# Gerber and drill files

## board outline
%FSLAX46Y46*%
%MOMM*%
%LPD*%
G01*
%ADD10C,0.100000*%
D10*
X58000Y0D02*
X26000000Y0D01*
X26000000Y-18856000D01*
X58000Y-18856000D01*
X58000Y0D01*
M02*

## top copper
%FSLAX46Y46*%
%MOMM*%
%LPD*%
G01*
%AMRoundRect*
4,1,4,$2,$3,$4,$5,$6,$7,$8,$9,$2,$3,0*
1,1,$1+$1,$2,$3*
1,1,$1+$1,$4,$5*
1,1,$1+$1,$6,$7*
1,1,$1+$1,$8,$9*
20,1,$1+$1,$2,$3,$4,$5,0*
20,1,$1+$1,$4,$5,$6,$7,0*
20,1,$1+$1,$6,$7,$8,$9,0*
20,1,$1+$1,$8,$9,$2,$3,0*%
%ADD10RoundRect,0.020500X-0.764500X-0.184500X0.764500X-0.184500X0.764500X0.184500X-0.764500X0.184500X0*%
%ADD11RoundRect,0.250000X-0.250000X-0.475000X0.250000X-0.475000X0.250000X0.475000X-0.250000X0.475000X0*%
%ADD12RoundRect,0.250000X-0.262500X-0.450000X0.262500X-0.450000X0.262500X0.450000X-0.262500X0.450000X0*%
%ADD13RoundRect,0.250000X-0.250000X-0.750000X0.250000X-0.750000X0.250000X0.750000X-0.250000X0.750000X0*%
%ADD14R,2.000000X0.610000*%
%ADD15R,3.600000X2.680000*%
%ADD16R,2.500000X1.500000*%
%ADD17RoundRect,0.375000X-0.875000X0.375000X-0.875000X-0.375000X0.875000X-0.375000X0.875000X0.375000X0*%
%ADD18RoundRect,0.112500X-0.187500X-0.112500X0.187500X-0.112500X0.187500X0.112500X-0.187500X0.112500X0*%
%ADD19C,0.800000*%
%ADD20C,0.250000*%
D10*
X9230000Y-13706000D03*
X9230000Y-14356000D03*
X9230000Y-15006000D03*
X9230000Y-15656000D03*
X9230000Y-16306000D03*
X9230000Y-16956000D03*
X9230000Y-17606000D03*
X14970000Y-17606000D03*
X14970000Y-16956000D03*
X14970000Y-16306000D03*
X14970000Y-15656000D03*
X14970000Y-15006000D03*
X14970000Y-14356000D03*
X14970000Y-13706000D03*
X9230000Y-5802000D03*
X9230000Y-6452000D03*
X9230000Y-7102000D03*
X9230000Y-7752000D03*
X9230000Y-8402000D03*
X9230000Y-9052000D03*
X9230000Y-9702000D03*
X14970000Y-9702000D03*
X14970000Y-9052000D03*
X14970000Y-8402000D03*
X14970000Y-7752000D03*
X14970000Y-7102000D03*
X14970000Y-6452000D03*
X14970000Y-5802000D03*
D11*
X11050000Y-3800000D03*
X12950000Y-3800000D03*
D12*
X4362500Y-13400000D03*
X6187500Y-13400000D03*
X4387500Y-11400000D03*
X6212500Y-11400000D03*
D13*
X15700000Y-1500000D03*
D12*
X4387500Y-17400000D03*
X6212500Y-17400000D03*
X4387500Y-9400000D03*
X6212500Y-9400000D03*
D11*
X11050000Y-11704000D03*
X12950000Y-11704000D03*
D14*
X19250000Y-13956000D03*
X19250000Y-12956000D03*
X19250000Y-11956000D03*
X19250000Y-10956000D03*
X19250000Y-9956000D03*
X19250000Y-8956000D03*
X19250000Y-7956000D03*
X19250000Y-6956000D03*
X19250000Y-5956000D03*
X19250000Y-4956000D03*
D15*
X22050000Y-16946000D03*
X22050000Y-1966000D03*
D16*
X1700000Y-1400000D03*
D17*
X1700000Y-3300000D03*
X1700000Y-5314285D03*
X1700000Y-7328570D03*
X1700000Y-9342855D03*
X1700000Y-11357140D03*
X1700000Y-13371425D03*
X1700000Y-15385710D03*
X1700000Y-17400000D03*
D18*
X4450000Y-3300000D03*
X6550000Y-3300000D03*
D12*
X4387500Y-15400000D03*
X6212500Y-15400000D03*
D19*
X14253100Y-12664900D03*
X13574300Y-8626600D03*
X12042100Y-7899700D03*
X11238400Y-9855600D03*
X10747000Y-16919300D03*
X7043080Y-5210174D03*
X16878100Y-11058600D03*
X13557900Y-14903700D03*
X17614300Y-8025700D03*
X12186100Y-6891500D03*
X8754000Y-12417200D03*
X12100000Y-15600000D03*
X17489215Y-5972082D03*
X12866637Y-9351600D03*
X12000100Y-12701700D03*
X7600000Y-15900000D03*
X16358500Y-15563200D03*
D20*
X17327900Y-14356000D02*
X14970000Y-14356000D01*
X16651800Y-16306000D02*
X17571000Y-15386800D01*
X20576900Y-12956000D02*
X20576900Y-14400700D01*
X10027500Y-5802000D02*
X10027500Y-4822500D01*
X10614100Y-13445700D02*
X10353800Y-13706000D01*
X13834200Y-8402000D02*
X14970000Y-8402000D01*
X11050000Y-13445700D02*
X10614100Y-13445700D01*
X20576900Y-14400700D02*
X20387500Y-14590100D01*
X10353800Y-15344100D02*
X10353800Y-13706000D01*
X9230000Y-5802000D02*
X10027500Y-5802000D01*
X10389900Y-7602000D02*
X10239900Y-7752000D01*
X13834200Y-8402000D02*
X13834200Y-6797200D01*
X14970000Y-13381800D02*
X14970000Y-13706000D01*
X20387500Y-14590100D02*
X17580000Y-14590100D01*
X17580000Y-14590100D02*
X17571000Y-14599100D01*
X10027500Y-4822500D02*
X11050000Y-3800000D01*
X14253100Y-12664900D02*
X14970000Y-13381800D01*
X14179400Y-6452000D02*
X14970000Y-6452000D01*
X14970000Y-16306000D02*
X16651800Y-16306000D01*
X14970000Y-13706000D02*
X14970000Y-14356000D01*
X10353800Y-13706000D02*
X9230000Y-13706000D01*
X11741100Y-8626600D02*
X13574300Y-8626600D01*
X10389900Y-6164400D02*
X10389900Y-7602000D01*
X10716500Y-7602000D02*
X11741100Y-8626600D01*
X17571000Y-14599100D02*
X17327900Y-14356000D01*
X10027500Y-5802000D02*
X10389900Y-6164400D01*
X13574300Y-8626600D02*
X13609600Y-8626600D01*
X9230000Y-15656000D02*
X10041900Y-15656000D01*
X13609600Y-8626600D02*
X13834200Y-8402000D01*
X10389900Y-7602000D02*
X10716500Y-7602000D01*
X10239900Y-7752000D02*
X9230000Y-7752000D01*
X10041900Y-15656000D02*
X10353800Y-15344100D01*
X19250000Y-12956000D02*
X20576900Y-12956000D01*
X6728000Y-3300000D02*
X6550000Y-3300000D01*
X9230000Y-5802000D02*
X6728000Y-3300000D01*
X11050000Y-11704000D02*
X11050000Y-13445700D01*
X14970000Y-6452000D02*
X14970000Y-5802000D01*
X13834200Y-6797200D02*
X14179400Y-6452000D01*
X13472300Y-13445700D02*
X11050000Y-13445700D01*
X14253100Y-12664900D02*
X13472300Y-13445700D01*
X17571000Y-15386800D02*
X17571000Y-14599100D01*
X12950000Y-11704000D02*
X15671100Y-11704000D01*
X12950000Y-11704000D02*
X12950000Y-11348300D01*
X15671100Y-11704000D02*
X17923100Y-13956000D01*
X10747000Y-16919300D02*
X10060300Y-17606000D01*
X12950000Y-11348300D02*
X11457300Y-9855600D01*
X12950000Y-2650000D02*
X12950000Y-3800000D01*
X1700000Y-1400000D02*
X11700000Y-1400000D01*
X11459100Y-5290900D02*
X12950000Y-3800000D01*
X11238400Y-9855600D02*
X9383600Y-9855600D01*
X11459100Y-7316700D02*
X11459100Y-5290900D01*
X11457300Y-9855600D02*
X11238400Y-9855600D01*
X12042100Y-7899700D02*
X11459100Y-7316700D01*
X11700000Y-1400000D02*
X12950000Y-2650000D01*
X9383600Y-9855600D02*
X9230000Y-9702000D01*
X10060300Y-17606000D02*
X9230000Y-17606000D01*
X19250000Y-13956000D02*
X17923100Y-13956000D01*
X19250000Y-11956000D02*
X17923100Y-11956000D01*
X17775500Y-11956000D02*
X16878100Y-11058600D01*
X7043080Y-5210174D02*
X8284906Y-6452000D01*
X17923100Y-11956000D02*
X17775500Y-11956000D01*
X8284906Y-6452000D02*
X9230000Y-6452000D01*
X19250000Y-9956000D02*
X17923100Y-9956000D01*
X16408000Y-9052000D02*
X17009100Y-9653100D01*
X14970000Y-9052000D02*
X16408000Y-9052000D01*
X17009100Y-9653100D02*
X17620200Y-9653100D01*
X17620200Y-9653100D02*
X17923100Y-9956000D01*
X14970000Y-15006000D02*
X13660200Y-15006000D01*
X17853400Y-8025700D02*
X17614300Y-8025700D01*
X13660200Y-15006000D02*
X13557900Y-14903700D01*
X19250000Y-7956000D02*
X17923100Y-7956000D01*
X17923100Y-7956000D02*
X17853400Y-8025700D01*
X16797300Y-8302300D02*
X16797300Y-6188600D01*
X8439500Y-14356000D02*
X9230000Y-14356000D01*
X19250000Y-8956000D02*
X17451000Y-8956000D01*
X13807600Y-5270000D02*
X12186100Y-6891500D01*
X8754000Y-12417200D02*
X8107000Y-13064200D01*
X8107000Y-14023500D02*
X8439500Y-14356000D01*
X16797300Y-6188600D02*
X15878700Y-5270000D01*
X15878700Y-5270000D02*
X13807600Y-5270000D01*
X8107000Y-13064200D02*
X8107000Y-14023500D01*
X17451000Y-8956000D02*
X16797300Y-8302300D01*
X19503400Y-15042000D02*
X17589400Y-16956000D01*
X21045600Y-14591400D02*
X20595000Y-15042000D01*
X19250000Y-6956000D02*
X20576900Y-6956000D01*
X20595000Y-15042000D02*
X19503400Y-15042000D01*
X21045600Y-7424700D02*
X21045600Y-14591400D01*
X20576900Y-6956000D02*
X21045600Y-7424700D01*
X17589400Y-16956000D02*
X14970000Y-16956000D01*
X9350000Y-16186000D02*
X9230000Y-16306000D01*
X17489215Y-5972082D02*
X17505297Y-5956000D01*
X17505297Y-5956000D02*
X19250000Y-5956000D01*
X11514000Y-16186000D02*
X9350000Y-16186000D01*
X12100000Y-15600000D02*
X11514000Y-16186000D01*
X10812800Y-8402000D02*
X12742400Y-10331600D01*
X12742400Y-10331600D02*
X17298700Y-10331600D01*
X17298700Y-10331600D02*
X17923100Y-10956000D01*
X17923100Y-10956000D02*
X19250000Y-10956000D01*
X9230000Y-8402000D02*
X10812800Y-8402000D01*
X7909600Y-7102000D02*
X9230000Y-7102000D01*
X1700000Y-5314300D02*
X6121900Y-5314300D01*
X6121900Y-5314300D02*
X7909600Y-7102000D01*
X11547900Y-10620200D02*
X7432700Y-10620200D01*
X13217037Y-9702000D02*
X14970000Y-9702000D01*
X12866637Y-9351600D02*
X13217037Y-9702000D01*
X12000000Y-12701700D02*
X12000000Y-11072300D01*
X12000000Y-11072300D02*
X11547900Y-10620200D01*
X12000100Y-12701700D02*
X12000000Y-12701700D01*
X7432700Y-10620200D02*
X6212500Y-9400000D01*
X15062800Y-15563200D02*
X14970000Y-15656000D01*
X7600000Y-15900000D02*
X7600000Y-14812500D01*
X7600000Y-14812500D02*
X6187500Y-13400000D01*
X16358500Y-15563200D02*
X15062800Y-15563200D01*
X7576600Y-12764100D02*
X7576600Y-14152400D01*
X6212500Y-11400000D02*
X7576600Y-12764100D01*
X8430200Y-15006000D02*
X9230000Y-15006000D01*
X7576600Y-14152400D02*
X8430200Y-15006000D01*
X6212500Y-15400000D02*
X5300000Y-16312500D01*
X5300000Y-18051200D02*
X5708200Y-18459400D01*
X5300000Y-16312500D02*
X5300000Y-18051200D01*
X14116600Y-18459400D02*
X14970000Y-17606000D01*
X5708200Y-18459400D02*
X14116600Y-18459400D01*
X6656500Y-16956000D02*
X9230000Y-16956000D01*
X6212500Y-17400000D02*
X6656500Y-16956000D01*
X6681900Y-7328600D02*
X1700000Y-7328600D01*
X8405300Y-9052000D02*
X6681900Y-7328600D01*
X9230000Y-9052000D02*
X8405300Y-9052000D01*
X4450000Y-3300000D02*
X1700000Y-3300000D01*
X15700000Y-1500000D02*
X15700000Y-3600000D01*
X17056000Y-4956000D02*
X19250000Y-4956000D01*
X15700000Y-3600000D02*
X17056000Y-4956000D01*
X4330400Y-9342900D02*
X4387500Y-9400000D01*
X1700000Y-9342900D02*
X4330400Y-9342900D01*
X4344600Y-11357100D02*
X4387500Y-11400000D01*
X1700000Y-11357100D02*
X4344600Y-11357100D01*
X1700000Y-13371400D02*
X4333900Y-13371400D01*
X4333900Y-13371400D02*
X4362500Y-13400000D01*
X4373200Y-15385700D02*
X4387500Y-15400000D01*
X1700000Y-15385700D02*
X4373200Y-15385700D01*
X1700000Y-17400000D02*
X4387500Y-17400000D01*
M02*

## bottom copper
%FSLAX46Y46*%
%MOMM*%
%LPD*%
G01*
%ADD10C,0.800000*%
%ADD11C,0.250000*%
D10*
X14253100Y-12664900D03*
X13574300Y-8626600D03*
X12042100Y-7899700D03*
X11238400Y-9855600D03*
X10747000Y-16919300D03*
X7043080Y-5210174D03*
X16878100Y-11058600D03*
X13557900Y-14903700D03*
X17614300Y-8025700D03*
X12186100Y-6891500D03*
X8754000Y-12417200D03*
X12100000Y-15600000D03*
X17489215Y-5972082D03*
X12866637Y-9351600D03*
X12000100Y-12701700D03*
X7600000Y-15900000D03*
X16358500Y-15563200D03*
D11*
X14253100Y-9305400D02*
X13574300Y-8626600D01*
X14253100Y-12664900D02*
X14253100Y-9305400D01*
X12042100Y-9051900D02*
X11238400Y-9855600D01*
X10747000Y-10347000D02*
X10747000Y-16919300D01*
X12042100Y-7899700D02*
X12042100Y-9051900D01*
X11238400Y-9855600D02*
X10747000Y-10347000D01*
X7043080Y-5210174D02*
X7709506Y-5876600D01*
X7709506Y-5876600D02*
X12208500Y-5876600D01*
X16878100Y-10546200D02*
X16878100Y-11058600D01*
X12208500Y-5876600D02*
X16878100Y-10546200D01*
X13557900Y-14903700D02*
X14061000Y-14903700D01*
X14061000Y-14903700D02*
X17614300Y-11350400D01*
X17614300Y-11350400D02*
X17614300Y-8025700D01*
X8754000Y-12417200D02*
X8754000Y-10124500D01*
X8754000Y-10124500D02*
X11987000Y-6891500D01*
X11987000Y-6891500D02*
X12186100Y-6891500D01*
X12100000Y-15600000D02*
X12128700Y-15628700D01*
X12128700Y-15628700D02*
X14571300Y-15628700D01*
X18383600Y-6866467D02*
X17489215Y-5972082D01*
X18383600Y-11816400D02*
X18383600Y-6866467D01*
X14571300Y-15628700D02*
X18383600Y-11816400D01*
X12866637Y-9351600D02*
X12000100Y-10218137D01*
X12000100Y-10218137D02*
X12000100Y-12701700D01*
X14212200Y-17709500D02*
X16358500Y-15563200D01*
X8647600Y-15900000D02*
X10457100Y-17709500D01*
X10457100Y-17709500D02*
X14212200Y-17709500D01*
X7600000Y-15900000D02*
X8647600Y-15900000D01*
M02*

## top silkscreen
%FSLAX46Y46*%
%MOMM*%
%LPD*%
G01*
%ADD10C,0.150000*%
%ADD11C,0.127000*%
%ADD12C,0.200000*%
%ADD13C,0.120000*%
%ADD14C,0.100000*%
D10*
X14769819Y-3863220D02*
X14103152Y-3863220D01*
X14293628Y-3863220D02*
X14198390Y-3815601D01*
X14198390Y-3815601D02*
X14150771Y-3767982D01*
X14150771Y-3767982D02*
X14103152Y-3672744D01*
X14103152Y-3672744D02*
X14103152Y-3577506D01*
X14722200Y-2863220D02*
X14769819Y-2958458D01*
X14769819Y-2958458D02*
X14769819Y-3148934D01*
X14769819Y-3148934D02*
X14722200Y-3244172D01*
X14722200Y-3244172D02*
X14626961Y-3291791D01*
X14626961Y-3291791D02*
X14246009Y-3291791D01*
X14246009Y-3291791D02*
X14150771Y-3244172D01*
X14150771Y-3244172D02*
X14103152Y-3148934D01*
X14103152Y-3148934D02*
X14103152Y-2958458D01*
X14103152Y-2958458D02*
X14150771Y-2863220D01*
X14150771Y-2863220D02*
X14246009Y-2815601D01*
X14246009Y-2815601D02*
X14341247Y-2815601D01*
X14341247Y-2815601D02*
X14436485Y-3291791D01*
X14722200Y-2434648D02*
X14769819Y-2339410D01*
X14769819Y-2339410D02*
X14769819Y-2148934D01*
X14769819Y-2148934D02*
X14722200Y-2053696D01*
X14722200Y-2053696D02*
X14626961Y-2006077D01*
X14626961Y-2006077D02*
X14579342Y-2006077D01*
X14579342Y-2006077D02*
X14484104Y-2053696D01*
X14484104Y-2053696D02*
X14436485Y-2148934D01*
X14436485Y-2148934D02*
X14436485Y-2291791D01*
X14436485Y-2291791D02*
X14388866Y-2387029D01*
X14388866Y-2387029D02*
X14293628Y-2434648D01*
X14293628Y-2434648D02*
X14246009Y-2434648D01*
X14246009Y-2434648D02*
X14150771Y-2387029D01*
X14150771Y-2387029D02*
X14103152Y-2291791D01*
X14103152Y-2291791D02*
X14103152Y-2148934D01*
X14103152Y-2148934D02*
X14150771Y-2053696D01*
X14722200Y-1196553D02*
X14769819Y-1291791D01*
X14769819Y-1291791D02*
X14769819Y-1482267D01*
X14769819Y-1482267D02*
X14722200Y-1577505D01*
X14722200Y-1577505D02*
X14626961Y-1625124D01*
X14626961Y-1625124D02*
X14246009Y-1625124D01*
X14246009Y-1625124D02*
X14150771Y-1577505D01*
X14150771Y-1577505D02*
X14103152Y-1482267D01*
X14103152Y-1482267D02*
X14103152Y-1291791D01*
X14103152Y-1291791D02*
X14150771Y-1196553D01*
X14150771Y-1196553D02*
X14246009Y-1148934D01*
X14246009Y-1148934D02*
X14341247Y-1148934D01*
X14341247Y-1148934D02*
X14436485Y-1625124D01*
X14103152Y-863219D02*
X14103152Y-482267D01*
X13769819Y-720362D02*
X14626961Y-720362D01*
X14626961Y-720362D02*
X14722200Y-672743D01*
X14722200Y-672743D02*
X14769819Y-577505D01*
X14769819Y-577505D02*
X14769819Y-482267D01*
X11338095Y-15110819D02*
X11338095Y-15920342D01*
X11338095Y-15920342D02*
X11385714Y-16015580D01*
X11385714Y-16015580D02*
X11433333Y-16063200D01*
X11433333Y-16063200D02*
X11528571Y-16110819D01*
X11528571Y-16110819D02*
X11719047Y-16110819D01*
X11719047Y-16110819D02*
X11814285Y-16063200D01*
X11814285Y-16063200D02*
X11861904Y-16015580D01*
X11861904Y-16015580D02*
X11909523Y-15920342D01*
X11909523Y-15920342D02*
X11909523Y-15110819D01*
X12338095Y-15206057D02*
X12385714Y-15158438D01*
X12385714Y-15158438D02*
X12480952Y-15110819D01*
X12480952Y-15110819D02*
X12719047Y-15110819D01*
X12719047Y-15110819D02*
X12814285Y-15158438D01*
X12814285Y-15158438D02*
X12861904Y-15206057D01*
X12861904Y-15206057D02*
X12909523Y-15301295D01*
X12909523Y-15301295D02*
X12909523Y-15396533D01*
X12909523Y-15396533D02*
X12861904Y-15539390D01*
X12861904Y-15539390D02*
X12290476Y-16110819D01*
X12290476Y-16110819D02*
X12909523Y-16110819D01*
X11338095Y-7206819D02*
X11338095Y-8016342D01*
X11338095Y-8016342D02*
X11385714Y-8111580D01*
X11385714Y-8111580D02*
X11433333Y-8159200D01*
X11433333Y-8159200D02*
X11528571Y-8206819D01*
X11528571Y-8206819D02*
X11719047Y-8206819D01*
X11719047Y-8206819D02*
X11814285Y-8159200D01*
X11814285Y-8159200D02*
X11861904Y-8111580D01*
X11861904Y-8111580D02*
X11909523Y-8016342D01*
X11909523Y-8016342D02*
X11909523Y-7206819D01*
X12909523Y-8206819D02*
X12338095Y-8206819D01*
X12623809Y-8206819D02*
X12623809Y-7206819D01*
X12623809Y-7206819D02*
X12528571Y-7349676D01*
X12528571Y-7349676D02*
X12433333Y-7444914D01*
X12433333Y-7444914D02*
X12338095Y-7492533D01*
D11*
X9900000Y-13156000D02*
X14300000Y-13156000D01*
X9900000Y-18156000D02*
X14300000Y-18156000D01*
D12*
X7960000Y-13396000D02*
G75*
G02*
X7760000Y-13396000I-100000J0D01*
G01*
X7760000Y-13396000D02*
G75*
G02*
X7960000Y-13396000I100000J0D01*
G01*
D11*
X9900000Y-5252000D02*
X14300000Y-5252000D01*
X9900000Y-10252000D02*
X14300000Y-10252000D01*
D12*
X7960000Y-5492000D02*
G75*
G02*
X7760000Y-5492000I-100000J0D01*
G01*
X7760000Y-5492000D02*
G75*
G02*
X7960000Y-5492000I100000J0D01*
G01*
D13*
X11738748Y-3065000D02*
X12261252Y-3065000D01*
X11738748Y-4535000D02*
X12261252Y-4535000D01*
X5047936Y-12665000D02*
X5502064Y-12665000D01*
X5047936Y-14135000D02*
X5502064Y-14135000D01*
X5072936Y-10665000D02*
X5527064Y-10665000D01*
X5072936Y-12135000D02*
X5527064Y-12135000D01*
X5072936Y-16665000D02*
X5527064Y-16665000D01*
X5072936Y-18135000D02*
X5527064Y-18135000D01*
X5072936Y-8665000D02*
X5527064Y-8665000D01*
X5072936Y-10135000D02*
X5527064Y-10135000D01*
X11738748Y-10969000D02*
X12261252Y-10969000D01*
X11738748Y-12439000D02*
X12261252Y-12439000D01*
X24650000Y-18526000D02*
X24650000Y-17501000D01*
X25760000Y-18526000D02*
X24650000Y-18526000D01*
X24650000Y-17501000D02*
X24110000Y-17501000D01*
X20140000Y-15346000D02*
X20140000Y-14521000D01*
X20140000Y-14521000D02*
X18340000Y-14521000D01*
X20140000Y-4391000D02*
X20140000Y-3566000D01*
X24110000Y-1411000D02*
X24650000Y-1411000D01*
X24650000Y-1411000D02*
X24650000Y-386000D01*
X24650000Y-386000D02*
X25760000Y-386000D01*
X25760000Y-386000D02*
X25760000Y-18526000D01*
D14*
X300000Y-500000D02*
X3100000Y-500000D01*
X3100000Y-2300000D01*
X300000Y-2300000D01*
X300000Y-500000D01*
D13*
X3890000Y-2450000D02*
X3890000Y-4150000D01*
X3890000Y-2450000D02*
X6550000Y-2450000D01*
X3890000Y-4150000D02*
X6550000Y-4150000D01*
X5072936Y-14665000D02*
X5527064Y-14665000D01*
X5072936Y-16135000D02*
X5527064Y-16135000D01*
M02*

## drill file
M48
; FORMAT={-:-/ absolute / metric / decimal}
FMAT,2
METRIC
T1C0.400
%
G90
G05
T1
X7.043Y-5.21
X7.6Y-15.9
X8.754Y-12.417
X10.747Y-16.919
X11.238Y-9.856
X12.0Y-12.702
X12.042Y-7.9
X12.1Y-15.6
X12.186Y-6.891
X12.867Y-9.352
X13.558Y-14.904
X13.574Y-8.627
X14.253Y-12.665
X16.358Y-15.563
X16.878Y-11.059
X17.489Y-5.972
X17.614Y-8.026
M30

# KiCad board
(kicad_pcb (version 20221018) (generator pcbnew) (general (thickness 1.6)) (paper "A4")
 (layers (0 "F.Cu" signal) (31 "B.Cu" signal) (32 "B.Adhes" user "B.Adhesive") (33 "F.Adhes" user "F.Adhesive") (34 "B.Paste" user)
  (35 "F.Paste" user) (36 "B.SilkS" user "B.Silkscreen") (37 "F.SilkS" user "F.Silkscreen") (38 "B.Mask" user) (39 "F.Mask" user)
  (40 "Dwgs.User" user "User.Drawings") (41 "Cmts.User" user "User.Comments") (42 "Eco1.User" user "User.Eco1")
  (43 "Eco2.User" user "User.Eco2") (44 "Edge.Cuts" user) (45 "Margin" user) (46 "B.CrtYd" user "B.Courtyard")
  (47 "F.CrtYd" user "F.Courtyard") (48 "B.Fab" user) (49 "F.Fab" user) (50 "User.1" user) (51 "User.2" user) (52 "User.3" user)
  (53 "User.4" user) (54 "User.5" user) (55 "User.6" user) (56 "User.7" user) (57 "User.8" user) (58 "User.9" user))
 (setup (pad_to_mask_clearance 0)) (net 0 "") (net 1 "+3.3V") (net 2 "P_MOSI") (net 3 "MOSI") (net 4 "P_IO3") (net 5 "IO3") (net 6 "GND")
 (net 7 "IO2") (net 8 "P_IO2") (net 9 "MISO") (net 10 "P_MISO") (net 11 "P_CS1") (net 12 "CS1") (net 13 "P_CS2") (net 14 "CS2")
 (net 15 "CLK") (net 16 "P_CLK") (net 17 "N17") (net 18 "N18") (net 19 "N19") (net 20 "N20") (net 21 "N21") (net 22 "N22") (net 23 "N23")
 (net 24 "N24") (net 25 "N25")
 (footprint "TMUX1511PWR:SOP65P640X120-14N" (layer "F.Cu") (at 12.1 15.656)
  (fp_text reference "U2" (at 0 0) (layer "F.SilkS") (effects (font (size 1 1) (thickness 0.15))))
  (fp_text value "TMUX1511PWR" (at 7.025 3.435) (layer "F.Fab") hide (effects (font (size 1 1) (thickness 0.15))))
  (fp_line (start -2.2 -2.5) (end 2.2 -2.5) (stroke (width 0.127) (type solid)) (layer "F.SilkS"))
  (fp_line (start -2.2 2.5) (end 2.2 2.5) (stroke (width 0.127) (type solid)) (layer "F.SilkS"))
  (fp_circle (center -4.24 -2.26) (end -4.14 -2.26) (stroke (width 0.2) (type solid)) (fill none) (layer "F.SilkS"))
  (pad "1" smd roundrect (at -2.87 -1.95) (size 1.57 0.41) (layers "F.Cu" "F.Paste" "F.Mask") (roundrect_rratio 0.05) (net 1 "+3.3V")
   (solder_mask_margin 0.102))
  (pad "2" smd roundrect (at -2.87 -1.3) (size 1.57 0.41) (layers "F.Cu" "F.Paste" "F.Mask") (roundrect_rratio 0.05) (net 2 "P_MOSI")
   (solder_mask_margin 0.102))
  (pad "3" smd roundrect (at -2.87 -0.65) (size 1.57 0.41) (layers "F.Cu" "F.Paste" "F.Mask") (roundrect_rratio 0.05) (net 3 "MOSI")
   (solder_mask_margin 0.102))
  (pad "4" smd roundrect (at -2.87 0) (size 1.57 0.41) (layers "F.Cu" "F.Paste" "F.Mask") (roundrect_rratio 0.05) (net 1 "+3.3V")
   (solder_mask_margin 0.102))
  (pad "5" smd roundrect (at -2.87 0.65) (size 1.57 0.41) (layers "F.Cu" "F.Paste" "F.Mask") (roundrect_rratio 0.05) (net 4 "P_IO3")
   (solder_mask_margin 0.102))
  (pad "6" smd roundrect (at -2.87 1.3) (size 1.57 0.41) (layers "F.Cu" "F.Paste" "F.Mask") (roundrect_rratio 0.05) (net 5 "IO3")
   (solder_mask_margin 0.102))
  (pad "7" smd roundrect (at -2.87 1.95) (size 1.57 0.41) (layers "F.Cu" "F.Paste" "F.Mask") (roundrect_rratio 0.05) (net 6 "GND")
   (solder_mask_margin 0.102))
  (pad "8" smd roundrect (at 2.87 1.95) (size 1.57 0.41) (layers "F.Cu" "F.Paste" "F.Mask") (roundrect_rratio 0.05) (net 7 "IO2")
   (solder_mask_margin 0.102))
  (pad "9" smd roundrect (at 2.87 1.3) (size 1.57 0.41) (layers "F.Cu" "F.Paste" "F.Mask") (roundrect_rratio 0.05) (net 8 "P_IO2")
   (solder_mask_margin 0.102))
  (pad "10" smd roundrect (at 2.87 0.65) (size 1.57 0.41) (layers "F.Cu" "F.Paste" "F.Mask") (roundrect_rratio 0.05) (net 1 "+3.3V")
   (solder_mask_margin 0.102))
  (pad "11" smd roundrect (at 2.87 0) (size 1.57 0.41) (layers "F.Cu" "F.Paste" "F.Mask") (roundrect_rratio 0.05) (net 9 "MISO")
   (solder_mask_margin 0.102))
  (pad "12" smd roundrect (at 2.87 -0.65) (size 1.57 0.41) (layers "F.Cu" "F.Paste" "F.Mask") (roundrect_rratio 0.05) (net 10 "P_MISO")
   (solder_mask_margin 0.102))
  (pad "13" smd roundrect (at 2.87 -1.3) (size 1.57 0.41) (layers "F.Cu" "F.Paste" "F.Mask") (roundrect_rratio 0.05) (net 1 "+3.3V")
   (solder_mask_margin 0.102))
  (pad "14" smd roundrect (at 2.87 -1.95) (size 1.57 0.41) (layers "F.Cu" "F.Paste" "F.Mask") (roundrect_rratio 0.05) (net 1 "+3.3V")
   (solder_mask_margin 0.102)))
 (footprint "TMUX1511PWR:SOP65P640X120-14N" (layer "F.Cu") (at 12.1 7.752)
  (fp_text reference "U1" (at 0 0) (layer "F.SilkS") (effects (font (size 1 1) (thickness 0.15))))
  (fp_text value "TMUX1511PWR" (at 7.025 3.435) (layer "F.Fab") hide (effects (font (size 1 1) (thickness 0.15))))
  (fp_line (start -2.2 -2.5) (end 2.2 -2.5) (stroke (width 0.127) (type solid)) (layer "F.SilkS"))
  (fp_line (start -2.2 2.5) (end 2.2 2.5) (stroke (width 0.127) (type solid)) (layer "F.SilkS"))
  (fp_circle (center -4.24 -2.26) (end -4.14 -2.26) (stroke (width 0.2) (type solid)) (fill none) (layer "F.SilkS"))
  (pad "1" smd roundrect (at -2.87 -1.95) (size 1.57 0.41) (layers "F.Cu" "F.Paste" "F.Mask") (roundrect_rratio 0.05) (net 1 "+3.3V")
   (solder_mask_margin 0.102))
  (pad "2" smd roundrect (at -2.87 -1.3) (size 1.57 0.41) (layers "F.Cu" "F.Paste" "F.Mask") (roundrect_rratio 0.05) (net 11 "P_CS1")
   (solder_mask_margin 0.102))
  (pad "3" smd roundrect (at -2.87 -0.65) (size 1.57 0.41) (layers "F.Cu" "F.Paste" "F.Mask") (roundrect_rratio 0.05) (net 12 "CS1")
   (solder_mask_margin 0.102))
  (pad "4" smd roundrect (at -2.87 0) (size 1.57 0.41) (layers "F.Cu" "F.Paste" "F.Mask") (roundrect_rratio 0.05) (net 1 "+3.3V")
   (solder_mask_margin 0.102))
  (pad "5" smd roundrect (at -2.87 0.65) (size 1.57 0.41) (layers "F.Cu" "F.Paste" "F.Mask") (roundrect_rratio 0.05) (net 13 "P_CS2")
   (solder_mask_margin 0.102))
  (pad "6" smd roundrect (at -2.87 1.3) (size 1.57 0.41) (layers "F.Cu" "F.Paste" "F.Mask") (roundrect_rratio 0.05) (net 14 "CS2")
   (solder_mask_margin 0.102))
  (pad "7" smd roundrect (at -2.87 1.95) (size 1.57 0.41) (layers "F.Cu" "F.Paste" "F.Mask") (roundrect_rratio 0.05) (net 6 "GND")
   (solder_mask_margin 0.102))
  (pad "8" smd roundrect (at 2.87 1.95) (size 1.57 0.41) (layers "F.Cu" "F.Paste" "F.Mask") (roundrect_rratio 0.05) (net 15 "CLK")
   (solder_mask_margin 0.102))
  (pad "9" smd roundrect (at 2.87 1.3) (size 1.57 0.41) (layers "F.Cu" "F.Paste" "F.Mask") (roundrect_rratio 0.05) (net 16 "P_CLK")
   (solder_mask_margin 0.102))
  (pad "10" smd roundrect (at 2.87 0.65) (size 1.57 0.41) (layers "F.Cu" "F.Paste" "F.Mask") (roundrect_rratio 0.05) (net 1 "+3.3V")
   (solder_mask_margin 0.102))
  (pad "11" smd roundrect (at 2.87 0) (size 1.57 0.41) (layers "F.Cu" "F.Paste" "F.Mask") (roundrect_rratio 0.05) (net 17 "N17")
   (solder_mask_margin 0.102))
  (pad "12" smd roundrect (at 2.87 -0.65) (size 1.57 0.41) (layers "F.Cu" "F.Paste" "F.Mask") (roundrect_rratio 0.05) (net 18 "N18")
   (solder_mask_margin 0.102))
  (pad "13" smd roundrect (at 2.87 -1.3) (size 1.57 0.41) (layers "F.Cu" "F.Paste" "F.Mask") (roundrect_rratio 0.05) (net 1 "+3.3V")
   (solder_mask_margin 0.102))
  (pad "14" smd roundrect (at 2.87 -1.95) (size 1.57 0.41) (layers "F.Cu" "F.Paste" "F.Mask") (roundrect_rratio 0.05) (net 1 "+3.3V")
   (solder_mask_margin 0.102)))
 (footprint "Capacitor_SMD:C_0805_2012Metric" (layer "F.Cu") (at 12 3.8)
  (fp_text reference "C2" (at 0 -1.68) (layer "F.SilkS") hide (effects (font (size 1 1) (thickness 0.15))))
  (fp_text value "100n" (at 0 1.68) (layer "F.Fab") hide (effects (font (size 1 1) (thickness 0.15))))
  (fp_line (start -0.261252 -0.735) (end 0.261252 -0.735) (stroke (width 0.12) (type solid)) (layer "F.SilkS"))
  (fp_line (start -0.261252 0.735) (end 0.261252 0.735) (stroke (width 0.12) (type solid)) (layer "F.SilkS"))
  (pad "1" smd roundrect (at -0.95 0) (size 1 1.45) (layers "F.Cu" "F.Paste" "F.Mask") (roundrect_rratio 0.25) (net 1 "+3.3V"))
  (pad "2" smd roundrect (at 0.95 0) (size 1 1.45) (layers "F.Cu" "F.Paste" "F.Mask") (roundrect_rratio 0.25) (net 6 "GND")))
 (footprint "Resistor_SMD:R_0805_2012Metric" (layer "F.Cu") (at 5.275 13.4)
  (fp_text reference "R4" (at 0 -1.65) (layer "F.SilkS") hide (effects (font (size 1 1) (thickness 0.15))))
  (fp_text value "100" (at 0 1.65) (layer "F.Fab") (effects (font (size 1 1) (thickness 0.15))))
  (fp_line (start -0.227064 -0.735) (end 0.227064 -0.735) (stroke (width 0.12) (type solid)) (layer "F.SilkS"))
  (fp_line (start -0.227064 0.735) (end 0.227064 0.735) (stroke (width 0.12) (type solid)) (layer "F.SilkS"))
  (pad "1" smd roundrect (at -0.9125 0) (size 1.025 1.4) (layers "F.Cu" "F.Paste" "F.Mask") (roundrect_rratio 0.243902439) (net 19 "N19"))
  (pad "2" smd roundrect (at 0.9125 0) (size 1.025 1.4) (layers "F.Cu" "F.Paste" "F.Mask") (roundrect_rratio 0.243902439) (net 9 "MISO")))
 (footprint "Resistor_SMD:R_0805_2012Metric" (layer "F.Cu") (at 5.3 11.4)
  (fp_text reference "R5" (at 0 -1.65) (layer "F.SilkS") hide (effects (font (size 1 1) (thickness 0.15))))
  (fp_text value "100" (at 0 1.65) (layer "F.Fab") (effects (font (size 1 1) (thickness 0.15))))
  (fp_line (start -0.227064 -0.735) (end 0.227064 -0.735) (stroke (width 0.12) (type solid)) (layer "F.SilkS"))
  (fp_line (start -0.227064 0.735) (end 0.227064 0.735) (stroke (width 0.12) (type solid)) (layer "F.SilkS"))
  (pad "1" smd roundrect (at -0.9125 0) (size 1.025 1.4) (layers "F.Cu" "F.Paste" "F.Mask") (roundrect_rratio 0.243902439) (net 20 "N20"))
  (pad "2" smd roundrect (at 0.9125 0) (size 1.025 1.4) (layers "F.Cu" "F.Paste" "F.Mask") (roundrect_rratio 0.243902439) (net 3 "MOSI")))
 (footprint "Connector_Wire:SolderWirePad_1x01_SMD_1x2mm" (layer "F.Cu") (at 15.7 1.5)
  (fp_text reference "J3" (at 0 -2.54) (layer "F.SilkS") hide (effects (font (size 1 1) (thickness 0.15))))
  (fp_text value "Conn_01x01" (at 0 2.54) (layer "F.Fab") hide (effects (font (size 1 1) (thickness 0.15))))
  (pad "1" smd roundrect (at 0 0) (size 1 2) (layers "F.Cu" "F.Paste" "F.Mask") (roundrect_rratio 0.25) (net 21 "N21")))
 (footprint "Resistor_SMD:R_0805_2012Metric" (layer "F.Cu") (at 5.3 17.4)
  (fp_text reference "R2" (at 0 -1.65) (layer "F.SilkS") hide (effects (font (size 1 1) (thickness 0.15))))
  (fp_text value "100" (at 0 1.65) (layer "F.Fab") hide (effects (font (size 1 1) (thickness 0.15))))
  (fp_line (start -0.227064 -0.735) (end 0.227064 -0.735) (stroke (width 0.12) (type solid)) (layer "F.SilkS"))
  (fp_line (start -0.227064 0.735) (end 0.227064 0.735) (stroke (width 0.12) (type solid)) (layer "F.SilkS"))
  (pad "1" smd roundrect (at -0.9125 0) (size 1.025 1.4) (layers "F.Cu" "F.Paste" "F.Mask") (roundrect_rratio 0.243902439) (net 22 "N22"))
  (pad "2" smd roundrect (at 0.9125 0) (size 1.025 1.4) (layers "F.Cu" "F.Paste" "F.Mask") (roundrect_rratio 0.243902439) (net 5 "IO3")))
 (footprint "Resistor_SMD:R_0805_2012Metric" (layer "F.Cu") (at 5.3 9.4)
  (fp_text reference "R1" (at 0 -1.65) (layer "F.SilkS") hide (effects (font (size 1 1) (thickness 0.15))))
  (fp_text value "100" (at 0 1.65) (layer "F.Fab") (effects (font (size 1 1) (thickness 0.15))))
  (fp_line (start -0.227064 -0.735) (end 0.227064 -0.735) (stroke (width 0.12) (type solid)) (layer "F.SilkS"))
  (fp_line (start -0.227064 0.735) (end 0.227064 0.735) (stroke (width 0.12) (type solid)) (layer "F.SilkS"))
  (pad "1" smd roundrect (at -0.9125 0) (size 1.025 1.4) (layers "F.Cu" "F.Paste" "F.Mask") (roundrect_rratio 0.243902439) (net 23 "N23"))
  (pad "2" smd roundrect (at 0.9125 0) (size 1.025 1.4) (layers "F.Cu" "F.Paste" "F.Mask") (roundrect_rratio 0.243902439) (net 15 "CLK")))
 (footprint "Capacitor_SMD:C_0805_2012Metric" (layer "F.Cu") (at 12 11.704)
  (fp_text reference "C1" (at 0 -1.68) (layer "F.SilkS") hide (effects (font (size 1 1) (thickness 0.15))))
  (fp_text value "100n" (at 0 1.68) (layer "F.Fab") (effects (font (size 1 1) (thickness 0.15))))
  (fp_line (start -0.261252 -0.735) (end 0.261252 -0.735) (stroke (width 0.12) (type solid)) (layer "F.SilkS"))
  (fp_line (start -0.261252 0.735) (end 0.261252 0.735) (stroke (width 0.12) (type solid)) (layer "F.SilkS"))
  (pad "1" smd roundrect (at -0.95 0) (size 1 1.45) (layers "F.Cu" "F.Paste" "F.Mask") (roundrect_rratio 0.25) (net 1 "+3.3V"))
  (pad "2" smd roundrect (at 0.95 0) (size 1 1.45) (layers "F.Cu" "F.Paste" "F.Mask") (roundrect_rratio 0.25) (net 6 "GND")))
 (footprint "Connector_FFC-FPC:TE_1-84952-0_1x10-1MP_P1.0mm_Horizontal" (layer "F.Cu") (at 21.05 9.456 90)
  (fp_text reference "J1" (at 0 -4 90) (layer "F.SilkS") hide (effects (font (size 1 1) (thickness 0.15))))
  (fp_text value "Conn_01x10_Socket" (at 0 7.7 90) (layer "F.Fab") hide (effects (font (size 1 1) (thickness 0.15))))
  (fp_line (start -9.07 3.6) (end -8.045 3.6) (stroke (width 0.12) (type solid)) (layer "F.SilkS"))
  (fp_line (start -9.07 4.71) (end -9.07 3.6) (stroke (width 0.12) (type solid)) (layer "F.SilkS"))
  (fp_line (start -8.045 3.6) (end -8.045 3.06) (stroke (width 0.12) (type solid)) (layer "F.SilkS"))
  (fp_line (start -5.89 -0.91) (end -5.065 -0.91) (stroke (width 0.12) (type solid)) (layer "F.SilkS"))
  (fp_line (start -5.065 -0.91) (end -5.065 -2.71) (stroke (width 0.12) (type solid)) (layer "F.SilkS"))
  (fp_line (start 5.065 -0.91) (end 5.89 -0.91) (stroke (width 0.12) (type solid)) (layer "F.SilkS"))
  (fp_line (start 8.045 3.06) (end 8.045 3.6) (stroke (width 0.12) (type solid)) (layer "F.SilkS"))
  (fp_line (start 8.045 3.6) (end 9.07 3.6) (stroke (width 0.12) (type solid)) (layer "F.SilkS"))
  (fp_line (start 9.07 3.6) (end 9.07 4.71) (stroke (width 0.12) (type solid)) (layer "F.SilkS"))
  (fp_line (start 9.07 4.71) (end -9.07 4.71) (stroke (width 0.12) (type solid)) (layer "F.SilkS"))
  (pad "1" smd rect (at -4.5 -1.8 90) (size 0.61 2) (layers "F.Cu" "F.Paste" "F.Mask") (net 6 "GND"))
  (pad "2" smd rect (at -3.5 -1.8 90) (size 0.61 2) (layers "F.Cu" "F.Paste" "F.Mask") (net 1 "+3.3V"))
  (pad "3" smd rect (at -2.5 -1.8 90) (size 0.61 2) (layers "F.Cu" "F.Paste" "F.Mask") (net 11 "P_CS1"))
  (pad "4" smd rect (at -1.5 -1.8 90) (size 0.61 2) (layers "F.Cu" "F.Paste" "F.Mask") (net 13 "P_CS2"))
  (pad "5" smd rect (at -0.5 -1.8 90) (size 0.61 2) (layers "F.Cu" "F.Paste" "F.Mask") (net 16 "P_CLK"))
  (pad "6" smd rect (at 0.5 -1.8 90) (size 0.61 2) (layers "F.Cu" "F.Paste" "F.Mask") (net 2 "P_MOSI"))
  (pad "7" smd rect (at 1.5 -1.8 90) (size 0.61 2) (layers "F.Cu" "F.Paste" "F.Mask") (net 10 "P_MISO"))
  (pad "8" smd rect (at 2.5 -1.8 90) (size 0.61 2) (layers "F.Cu" "F.Paste" "F.Mask") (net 8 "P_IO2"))
  (pad "9" smd rect (at 3.5 -1.8 90) (size 0.61 2) (layers "F.Cu" "F.Paste" "F.Mask") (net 4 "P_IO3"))
  (pad "10" smd rect (at 4.5 -1.8 90) (size 0.61 2) (layers "F.Cu" "F.Paste" "F.Mask") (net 21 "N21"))
  (pad "MP" smd rect (at -7.49 1 90) (size 2.68 3.6) (layers "F.Cu" "F.Paste" "F.Mask"))
  (pad "MP" smd rect (at 7.49 1 90) (size 2.68 3.6) (layers "F.Cu" "F.Paste" "F.Mask")))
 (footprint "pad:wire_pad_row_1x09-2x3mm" (layer "F.Cu") (at 1.7 1.4 -90)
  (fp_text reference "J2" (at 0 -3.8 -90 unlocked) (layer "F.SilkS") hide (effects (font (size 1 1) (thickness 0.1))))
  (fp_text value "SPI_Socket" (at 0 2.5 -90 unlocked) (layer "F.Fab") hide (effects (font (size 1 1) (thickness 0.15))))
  (fp_rect (start -0.9 -1.4) (end 0.9 1.4) (stroke (width 0.1) (type default)) (fill none) (layer "F.SilkS"))
  (pad "1" smd rect (at 0 0 270) (size 1.5 2.5) (layers "F.Cu" "F.Paste" "F.Mask") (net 6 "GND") (thermal_bridge_angle 45))
  (pad "2" smd roundrect (at 1.9 0 270) (size 1.5 2.5) (layers "F.Cu" "F.Paste" "F.Mask") (roundrect_rratio 0.25) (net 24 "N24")
   (thermal_bridge_angle 45))
  (pad "3" smd roundrect (at 3.914285 0 270) (size 1.5 2.5) (layers "F.Cu" "F.Paste" "F.Mask") (roundrect_rratio 0.25) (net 12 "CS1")
   (thermal_bridge_angle 45))
  (pad "4" smd roundrect (at 5.92857 0 270) (size 1.5 2.5) (layers "F.Cu" "F.Paste" "F.Mask") (roundrect_rratio 0.25) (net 14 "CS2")
   (thermal_bridge_angle 45))
  (pad "5" smd roundrect (at 7.942855 0 270) (size 1.5 2.5) (layers "F.Cu" "F.Paste" "F.Mask") (roundrect_rratio 0.25) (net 23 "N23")
   (thermal_bridge_angle 45))
  (pad "6" smd roundrect (at 9.95714 0 270) (size 1.5 2.5) (layers "F.Cu" "F.Paste" "F.Mask") (roundrect_rratio 0.25) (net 20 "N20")
   (thermal_bridge_angle 45))
  (pad "7" smd roundrect (at 11.971425 0 270) (size 1.5 2.5) (layers "F.Cu" "F.Paste" "F.Mask") (roundrect_rratio 0.25) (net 19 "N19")
   (thermal_bridge_angle 45))
  (pad "8" smd roundrect (at 13.98571 0 270) (size 1.5 2.5) (layers "F.Cu" "F.Paste" "F.Mask") (roundrect_rratio 0.25) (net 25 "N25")
   (thermal_bridge_angle 45))
  (pad "9" smd roundrect (at 16 0 270) (size 1.5 2.5) (layers "F.Cu" "F.Paste" "F.Mask") (roundrect_rratio 0.25) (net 22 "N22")
   (thermal_bridge_angle 45)))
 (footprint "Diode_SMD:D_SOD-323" (layer "F.Cu") (at 5.5 3.3)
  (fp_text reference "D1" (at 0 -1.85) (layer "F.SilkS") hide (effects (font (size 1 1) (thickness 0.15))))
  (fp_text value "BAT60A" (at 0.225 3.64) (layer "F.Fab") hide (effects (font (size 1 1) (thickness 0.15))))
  (fp_line (start -1.61 -0.85) (end -1.61 0.85) (stroke (width 0.12) (type solid)) (layer "F.SilkS"))
  (fp_line (start -1.61 -0.85) (end 1.05 -0.85) (stroke (width 0.12) (type solid)) (layer "F.SilkS"))
  (fp_line (start -1.61 0.85) (end 1.05 0.85) (stroke (width 0.12) (type solid)) (layer "F.SilkS"))
  (pad "1" smd roundrect (at -1.05 0) (size 0.6 0.45) (layers "F.Cu" "F.Paste" "F.Mask") (roundrect_rratio 0.25) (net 24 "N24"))
  (pad "2" smd roundrect (at 1.05 0) (size 0.6 0.45) (layers "F.Cu" "F.Paste" "F.Mask") (roundrect_rratio 0.25) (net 1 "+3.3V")))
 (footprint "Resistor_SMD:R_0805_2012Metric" (layer "F.Cu") (at 5.3 15.4)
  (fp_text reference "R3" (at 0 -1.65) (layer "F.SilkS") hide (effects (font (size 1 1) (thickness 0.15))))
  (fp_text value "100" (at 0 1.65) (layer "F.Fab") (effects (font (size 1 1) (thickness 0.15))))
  (fp_line (start -0.227064 -0.735) (end 0.227064 -0.735) (stroke (width 0.12) (type solid)) (layer "F.SilkS"))
  (fp_line (start -0.227064 0.735) (end 0.227064 0.735) (stroke (width 0.12) (type solid)) (layer "F.SilkS"))
  (pad "1" smd roundrect (at -0.9125 0) (size 1.025 1.4) (layers "F.Cu" "F.Paste" "F.Mask") (roundrect_rratio 0.243902439) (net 25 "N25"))
  (pad "2" smd roundrect (at 0.9125 0) (size 1.025 1.4) (layers "F.Cu" "F.Paste" "F.Mask") (roundrect_rratio 0.243902439) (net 7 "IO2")))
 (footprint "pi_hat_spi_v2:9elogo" (layer "B.Cu") (at 21 14.9 180)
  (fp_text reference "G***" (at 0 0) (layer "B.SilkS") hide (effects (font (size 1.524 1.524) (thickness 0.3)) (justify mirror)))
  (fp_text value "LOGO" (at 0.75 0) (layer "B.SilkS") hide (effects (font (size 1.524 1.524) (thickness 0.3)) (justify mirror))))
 (gr_rect (start 0.058 0) (end 26 18.856) (stroke (width 0.1) (type default)) (fill none) (layer "Edge.Cuts"))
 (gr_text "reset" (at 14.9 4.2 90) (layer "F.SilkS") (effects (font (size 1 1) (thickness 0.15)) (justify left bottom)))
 (segment (start 17.3279 14.356) (end 14.97 14.356) (width 0.25) (layer "F.Cu") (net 1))
 (segment (start 16.6518 16.306) (end 17.571 15.3868) (width 0.25) (layer "F.Cu") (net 1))
 (segment (start 20.5769 12.956) (end 20.5769 14.4007) (width 0.25) (layer "F.Cu") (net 1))
 (segment (start 10.0275 5.802) (end 10.0275 4.8225) (width 0.25) (layer "F.Cu") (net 1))
 (segment (start 10.6141 13.4457) (end 10.3538 13.706) (width 0.25) (layer "F.Cu") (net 1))
 (segment (start 13.8342 8.402) (end 14.97 8.402) (width 0.25) (layer "F.Cu") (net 1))
 (segment (start 11.05 13.4457) (end 10.6141 13.4457) (width 0.25) (layer "F.Cu") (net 1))
 (segment (start 20.5769 14.4007) (end 20.3875 14.5901) (width 0.25) (layer "F.Cu") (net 1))
 (segment (start 10.3538 15.3441) (end 10.3538 13.706) (width 0.25) (layer "F.Cu") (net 1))
 (segment (start 9.23 5.802) (end 10.0275 5.802) (width 0.25) (layer "F.Cu") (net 1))
 (segment (start 10.3899 7.602) (end 10.2399 7.752) (width 0.25) (layer "F.Cu") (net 1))
 (segment (start 13.8342 8.402) (end 13.8342 6.7972) (width 0.25) (layer "F.Cu") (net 1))
 (segment (start 14.97 13.3818) (end 14.97 13.706) (width 0.25) (layer "F.Cu") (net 1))
 (segment (start 20.3875 14.5901) (end 17.58 14.5901) (width 0.25) (layer "F.Cu") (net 1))
 (segment (start 17.58 14.5901) (end 17.571 14.5991) (width 0.25) (layer "F.Cu") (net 1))
 (segment (start 10.0275 4.8225) (end 11.05 3.8) (width 0.25) (layer "F.Cu") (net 1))
 (segment (start 14.2531 12.6649) (end 14.97 13.3818) (width 0.25) (layer "F.Cu") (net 1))
 (segment (start 14.1794 6.452) (end 14.97 6.452) (width 0.25) (layer "F.Cu") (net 1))
 (segment (start 14.97 16.306) (end 16.6518 16.306) (width 0.25) (layer "F.Cu") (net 1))
 (segment (start 14.97 13.706) (end 14.97 14.356) (width 0.25) (layer "F.Cu") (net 1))
 (segment (start 10.3538 13.706) (end 9.23 13.706) (width 0.25) (layer "F.Cu") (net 1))
 (segment (start 11.7411 8.6266) (end 13.5743 8.6266) (width 0.25) (layer "F.Cu") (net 1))
 (segment (start 10.3899 6.1644) (end 10.3899 7.602) (width 0.25) (layer "F.Cu") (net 1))
 (segment (start 10.7165 7.602) (end 11.7411 8.6266) (width 0.25) (layer "F.Cu") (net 1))
 (segment (start 17.571 14.5991) (end 17.3279 14.356) (width 0.25) (layer "F.Cu") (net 1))
 (segment (start 10.0275 5.802) (end 10.3899 6.1644) (width 0.25) (layer "F.Cu") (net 1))
 (segment (start 13.5743 8.6266) (end 13.6096 8.6266) (width 0.25) (layer "F.Cu") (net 1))
 (segment (start 9.23 15.656) (end 10.0419 15.656) (width 0.25) (layer "F.Cu") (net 1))
 (segment (start 13.6096 8.6266) (end 13.8342 8.402) (width 0.25) (layer "F.Cu") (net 1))
 (segment (start 10.3899 7.602) (end 10.7165 7.602) (width 0.25) (layer "F.Cu") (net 1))
 (segment (start 10.2399 7.752) (end 9.23 7.752) (width 0.25) (layer "F.Cu") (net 1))
 (segment (start 10.0419 15.656) (end 10.3538 15.3441) (width 0.25) (layer "F.Cu") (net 1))
 (segment (start 19.25 12.956) (end 20.5769 12.956) (width 0.25) (layer "F.Cu") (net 1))
 (segment (start 6.728 3.3) (end 6.55 3.3) (width 0.25) (layer "F.Cu") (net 1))
 (segment (start 9.23 5.802) (end 6.728 3.3) (width 0.25) (layer "F.Cu") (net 1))
 (segment (start 11.05 11.704) (end 11.05 13.4457) (width 0.25) (layer "F.Cu") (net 1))
 (segment (start 14.97 6.452) (end 14.97 5.802) (width 0.25) (layer "F.Cu") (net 1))
 (segment (start 13.8342 6.7972) (end 14.1794 6.452) (width 0.25) (layer "F.Cu") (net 1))
 (segment (start 13.4723 13.4457) (end 11.05 13.4457) (width 0.25) (layer "F.Cu") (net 1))
 (segment (start 14.2531 12.6649) (end 13.4723 13.4457) (width 0.25) (layer "F.Cu") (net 1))
 (segment (start 17.571 15.3868) (end 17.571 14.5991) (width 0.25) (layer "F.Cu") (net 1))
 (via (at 14.2531 12.6649) (size 0.8) (drill 0.4) (layers "F.Cu" "B.Cu") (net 1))
 (via (at 13.5743 8.6266) (size 0.8) (drill 0.4) (layers "F.Cu" "B.Cu") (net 1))
 (segment (start 14.2531 9.3054) (end 13.5743 8.6266) (width 0.25) (layer "B.Cu") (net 1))
 (segment (start 14.2531 12.6649) (end 14.2531 9.3054) (width 0.25) (layer "B.Cu") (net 1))
 (segment (start 12.95 11.704) (end 15.6711 11.704) (width 0.25) (layer "F.Cu") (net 6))
 (segment (start 12.95 11.704) (end 12.95 11.3483) (width 0.25) (layer "F.Cu") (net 6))
 (segment (start 15.6711 11.704) (end 17.9231 13.956) (width 0.25) (layer "F.Cu") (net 6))
 (segment (start 10.747 16.9193) (end 10.0603 17.606) (width 0.25) (layer "F.Cu") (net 6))
 (segment (start 12.95 11.3483) (end 11.4573 9.8556) (width 0.25) (layer "F.Cu") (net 6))
 (segment (start 12.95 2.65) (end 12.95 3.8) (width 0.25) (layer "F.Cu") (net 6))
 (segment (start 1.7 1.4) (end 11.7 1.4) (width 0.25) (layer "F.Cu") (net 6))
 (segment (start 11.4591 5.2909) (end 12.95 3.8) (width 0.25) (layer "F.Cu") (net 6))
 (segment (start 11.2384 9.8556) (end 9.3836 9.8556) (width 0.25) (layer "F.Cu") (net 6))
 (segment (start 11.4591 7.3167) (end 11.4591 5.2909) (width 0.25) (layer "F.Cu") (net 6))
 (segment (start 11.4573 9.8556) (end 11.2384 9.8556) (width 0.25) (layer "F.Cu") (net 6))
 (segment (start 12.0421 7.8997) (end 11.4591 7.3167) (width 0.25) (layer "F.Cu") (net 6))
 (segment (start 11.7 1.4) (end 12.95 2.65) (width 0.25) (layer "F.Cu") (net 6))
 (segment (start 9.3836 9.8556) (end 9.23 9.702) (width 0.25) (layer "F.Cu") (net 6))
 (segment (start 10.0603 17.606) (end 9.23 17.606) (width 0.25) (layer "F.Cu") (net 6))
 (segment (start 19.25 13.956) (end 17.9231 13.956) (width 0.25) (layer "F.Cu") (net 6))
 (via (at 12.0421 7.8997) (size 0.8) (drill 0.4) (layers "F.Cu" "B.Cu") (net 6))
 (via (at 11.2384 9.8556) (size 0.8) (drill 0.4) (layers "F.Cu" "B.Cu") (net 6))
 (via (at 10.747 16.9193) (size 0.8) (drill 0.4) (layers "F.Cu" "B.Cu") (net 6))
 (segment (start 12.0421 9.0519) (end 11.2384 9.8556) (width 0.25) (layer "B.Cu") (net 6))
 (segment (start 10.747 10.347) (end 10.747 16.9193) (width 0.25) (layer "B.Cu") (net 6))
 (segment (start 12.0421 7.8997) (end 12.0421 9.0519) (width 0.25) (layer "B.Cu") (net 6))
 (segment (start 11.2384 9.8556) (end 10.747 10.347) (width 0.25) (layer "B.Cu") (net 6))
 (segment (start 19.25 11.956) (end 17.9231 11.956) (width 0.25) (layer "F.Cu") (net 11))
 (segment (start 17.7755 11.956) (end 16.8781 11.0586) (width 0.25) (layer "F.Cu") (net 11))
 (segment (start 7.04308 5.210174) (end 8.284906 6.452) (width 0.25) (layer "F.Cu") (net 11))
 (segment (start 17.9231 11.956) (end 17.7755 11.956) (width 0.25) (layer "F.Cu") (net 11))
 (segment (start 8.284906 6.452) (end 9.23 6.452) (width 0.25) (layer "F.Cu") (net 11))
 (via (at 7.04308 5.210174) (size 0.8) (drill 0.4) (layers "F.Cu" "B.Cu") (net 11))
 (via (at 16.8781 11.0586) (size 0.8) (drill 0.4) (layers "F.Cu" "B.Cu") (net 11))
 (segment (start 7.04308 5.210174) (end 7.709506 5.8766) (width 0.25) (layer "B.Cu") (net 11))
 (segment (start 7.709506 5.8766) (end 12.2085 5.8766) (width 0.25) (layer "B.Cu") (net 11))
 (segment (start 16.8781 10.5462) (end 16.8781 11.0586) (width 0.25) (layer "B.Cu") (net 11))
 (segment (start 12.2085 5.8766) (end 16.8781 10.5462) (width 0.25) (layer "B.Cu") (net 11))
 (segment (start 19.25 9.956) (end 17.9231 9.956) (width 0.25) (layer "F.Cu") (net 16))
 (segment (start 16.408 9.052) (end 17.0091 9.6531) (width 0.25) (layer "F.Cu") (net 16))
 (segment (start 14.97 9.052) (end 16.408 9.052) (width 0.25) (layer "F.Cu") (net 16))
 (segment (start 17.0091 9.6531) (end 17.6202 9.6531) (width 0.25) (layer "F.Cu") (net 16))
 (segment (start 17.6202 9.6531) (end 17.9231 9.956) (width 0.25) (layer "F.Cu") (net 16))
 (segment (start 14.97 15.006) (end 13.6602 15.006) (width 0.25) (layer "F.Cu") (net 10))
 (segment (start 17.8534 8.0257) (end 17.6143 8.0257) (width 0.25) (layer "F.Cu") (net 10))
 (segment (start 13.6602 15.006) (end 13.5579 14.9037) (width 0.25) (layer "F.Cu") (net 10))
 (segment (start 19.25 7.956) (end 17.9231 7.956) (width 0.25) (layer "F.Cu") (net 10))
 (segment (start 17.9231 7.956) (end 17.8534 8.0257) (width 0.25) (layer "F.Cu") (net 10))
 (via (at 13.5579 14.9037) (size 0.8) (drill 0.4) (layers "F.Cu" "B.Cu") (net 10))
 (via (at 17.6143 8.0257) (size 0.8) (drill 0.4) (layers "F.Cu" "B.Cu") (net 10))
 (segment (start 13.5579 14.9037) (end 14.061 14.9037) (width 0.25) (layer "B.Cu") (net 10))
 (segment (start 14.061 14.9037) (end 17.6143 11.3504) (width 0.25) (layer "B.Cu") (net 10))
 (segment (start 17.6143 11.3504) (end 17.6143 8.0257) (width 0.25) (layer "B.Cu") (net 10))
 (segment (start 16.7973 8.3023) (end 16.7973 6.1886) (width 0.25) (layer "F.Cu") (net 2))
 (segment (start 8.4395 14.356) (end 9.23 14.356) (width 0.25) (layer "F.Cu") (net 2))
 (segment (start 19.25 8.956) (end 17.451 8.956) (width 0.25) (layer "F.Cu") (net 2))
 (segment (start 13.8076 5.27) (end 12.1861 6.8915) (width 0.25) (layer "F.Cu") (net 2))
 (segment (start 8.754 12.4172) (end 8.107 13.0642) (width 0.25) (layer "F.Cu") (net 2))
 (segment (start 8.107 14.0235) (end 8.4395 14.356) (width 0.25) (layer "F.Cu") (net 2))
 (segment (start 16.7973 6.1886) (end 15.8787 5.27) (width 0.25) (layer "F.Cu") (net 2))
 (segment (start 15.8787 5.27) (end 13.8076 5.27) (width 0.25) (layer "F.Cu") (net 2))
 (segment (start 8.107 13.0642) (end 8.107 14.0235) (width 0.25) (layer "F.Cu") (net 2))
 (segment (start 17.451 8.956) (end 16.7973 8.3023) (width 0.25) (layer "F.Cu") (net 2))
 (via (at 12.1861 6.8915) (size 0.8) (drill 0.4) (layers "F.Cu" "B.Cu") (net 2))
 (via (at 8.754 12.4172) (size 0.8) (drill 0.4) (layers "F.Cu" "B.Cu") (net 2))
 (segment (start 8.754 12.4172) (end 8.754 10.1245) (width 0.25) (layer "B.Cu") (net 2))
 (segment (start 8.754 10.1245) (end 11.987 6.8915) (width 0.25) (layer "B.Cu") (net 2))
 (segment (start 11.987 6.8915) (end 12.1861 6.8915) (width 0.25) (layer "B.Cu") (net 2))
 (segment (start 19.5034 15.042) (end 17.5894 16.956) (width 0.25) (layer "F.Cu") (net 8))
 (segment (start 21.0456 14.5914) (end 20.595 15.042) (width 0.25) (layer "F.Cu") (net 8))
 (segment (start 19.25 6.956) (end 20.5769 6.956) (width 0.25) (layer "F.Cu") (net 8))
 (segment (start 20.595 15.042) (end 19.5034 15.042) (width 0.25) (layer "F.Cu") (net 8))
 (segment (start 21.0456 7.4247) (end 21.0456 14.5914) (width 0.25) (layer "F.Cu") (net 8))
 (segment (start 20.5769 6.956) (end 21.0456 7.4247) (width 0.25) (layer "F.Cu") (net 8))
 (segment (start 17.5894 16.956) (end 14.97 16.956) (width 0.25) (layer "F.Cu") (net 8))
 (segment (start 9.35 16.186) (end 9.23 16.306) (width 0.25) (layer "F.Cu") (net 4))
 (segment (start 17.489215 5.972082) (end 17.505297 5.956) (width 0.25) (layer "F.Cu") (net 4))
 (segment (start 17.505297 5.956) (end 19.25 5.956) (width 0.25) (layer "F.Cu") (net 4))
 (segment (start 11.514 16.186) (end 9.35 16.186) (width 0.25) (layer "F.Cu") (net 4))
 (segment (start 12.1 15.6) (end 11.514 16.186) (width 0.25) (layer "F.Cu") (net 4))
 (via (at 12.1 15.6) (size 0.8) (drill 0.4) (layers "F.Cu" "B.Cu") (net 4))
 (via (at 17.489215 5.972082) (size 0.8) (drill 0.4) (layers "F.Cu" "B.Cu") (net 4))
 (segment (start 12.1 15.6) (end 12.1287 15.6287) (width 0.25) (layer "B.Cu") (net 4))
 (segment (start 12.1287 15.6287) (end 14.5713 15.6287) (width 0.25) (layer "B.Cu") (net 4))
 (segment (start 18.3836 6.866467) (end 17.489215 5.972082) (width 0.25) (layer "B.Cu") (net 4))
 (segment (start 18.3836 11.8164) (end 18.3836 6.866467) (width 0.25) (layer "B.Cu") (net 4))
 (segment (start 14.5713 15.6287) (end 18.3836 11.8164) (width 0.25) (layer "B.Cu") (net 4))
 (segment (start 10.8128 8.402) (end 12.7424 10.3316) (width 0.25) (layer "F.Cu") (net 13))
 (segment (start 12.7424 10.3316) (end 17.2987 10.3316) (width 0.25) (layer "F.Cu") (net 13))
 (segment (start 17.2987 10.3316) (end 17.9231 10.956) (width 0.25) (layer "F.Cu") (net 13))
 (segment (start 17.9231 10.956) (end 19.25 10.956) (width 0.25) (layer "F.Cu") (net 13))
 (segment (start 9.23 8.402) (end 10.8128 8.402) (width 0.25) (layer "F.Cu") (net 13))
 (segment (start 7.9096 7.102) (end 9.23 7.102) (width 0.25) (layer "F.Cu") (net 12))
 (segment (start 1.7 5.3143) (end 6.1219 5.3143) (width 0.25) (layer "F.Cu") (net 12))
 (segment (start 6.1219 5.3143) (end 7.9096 7.102) (width 0.25) (layer "F.Cu") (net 12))
 (segment (start 11.5479 10.6202) (end 7.4327 10.6202) (width 0.25) (layer "F.Cu") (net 15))
 (segment (start 13.217037 9.702) (end 14.97 9.702) (width 0.25) (layer "F.Cu") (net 15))
 (segment (start 12.866637 9.3516) (end 13.217037 9.702) (width 0.25) (layer "F.Cu") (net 15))
 (segment (start 12 12.7017) (end 12 11.0723) (width 0.25) (layer "F.Cu") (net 15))
 (segment (start 12 11.0723) (end 11.5479 10.6202) (width 0.25) (layer "F.Cu") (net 15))
 (segment (start 12.0001 12.7017) (end 12 12.7017) (width 0.25) (layer "F.Cu") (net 15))
 (segment (start 7.4327 10.6202) (end 6.2125 9.4) (width 0.25) (layer "F.Cu") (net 15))
 (via (at 12.866637 9.3516) (size 0.8) (drill 0.4) (layers "F.Cu" "B.Cu") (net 15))
 (via (at 12.0001 12.7017) (size 0.8) (drill 0.4) (layers "F.Cu" "B.Cu") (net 15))
 (segment (start 12.866637 9.3516) (end 12.0001 10.218137) (width 0.25) (layer "B.Cu") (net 15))
 (segment (start 12.0001 10.218137) (end 12.0001 12.7017) (width 0.25) (layer "B.Cu") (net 15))
 (segment (start 15.0628 15.5632) (end 14.97 15.656) (width 0.25) (layer "F.Cu") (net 9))
 (segment (start 7.6 15.9) (end 7.6 14.8125) (width 0.25) (layer "F.Cu") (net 9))
 (segment (start 7.6 14.8125) (end 6.1875 13.4) (width 0.25) (layer "F.Cu") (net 9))
 (segment (start 16.3585 15.5632) (end 15.0628 15.5632) (width 0.25) (layer "F.Cu") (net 9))
 (via (at 7.6 15.9) (size 0.8) (drill 0.4) (layers "F.Cu" "B.Cu") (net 9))
 (via (at 16.3585 15.5632) (size 0.8) (drill 0.4) (layers "F.Cu" "B.Cu") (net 9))
 (segment (start 14.2122 17.7095) (end 16.3585 15.5632) (width 0.25) (layer "B.Cu") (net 9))
 (segment (start 8.6476 15.9) (end 10.4571 17.7095) (width 0.25) (layer "B.Cu") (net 9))
 (segment (start 10.4571 17.7095) (end 14.2122 17.7095) (width 0.25) (layer "B.Cu") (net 9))
 (segment (start 7.6 15.9) (end 8.6476 15.9) (width 0.25) (layer "B.Cu") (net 9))
 (segment (start 7.5766 12.7641) (end 7.5766 14.1524) (width 0.25) (layer "F.Cu") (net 3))
 (segment (start 6.2125 11.4) (end 7.5766 12.7641) (width 0.25) (layer "F.Cu") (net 3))
 (segment (start 8.4302 15.006) (end 9.23 15.006) (width 0.25) (layer "F.Cu") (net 3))
 (segment (start 7.5766 14.1524) (end 8.4302 15.006) (width 0.25) (layer "F.Cu") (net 3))
 (segment (start 6.2125 15.4) (end 5.3 16.3125) (width 0.25) (layer "F.Cu") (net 7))
 (segment (start 5.3 18.0512) (end 5.7082 18.4594) (width 0.25) (layer "F.Cu") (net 7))
 (segment (start 5.3 16.3125) (end 5.3 18.0512) (width 0.25) (layer "F.Cu") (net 7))
 (segment (start 14.1166 18.4594) (end 14.97 17.606) (width 0.25) (layer "F.Cu") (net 7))
 (segment (start 5.7082 18.4594) (end 14.1166 18.4594) (width 0.25) (layer "F.Cu") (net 7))
 (segment (start 6.6565 16.956) (end 9.23 16.956) (width 0.25) (layer "F.Cu") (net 5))
 (segment (start 6.2125 17.4) (end 6.6565 16.956) (width 0.25) (layer "F.Cu") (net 5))
 (segment (start 6.6819 7.3286) (end 1.7 7.3286) (width 0.25) (layer "F.Cu") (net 14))
 (segment (start 8.4053 9.052) (end 6.6819 7.3286) (width 0.25) (layer "F.Cu") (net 14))
 (segment (start 9.23 9.052) (end 8.4053 9.052) (width 0.25) (layer "F.Cu") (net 14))
 (segment (start 4.45 3.3) (end 1.7 3.3) (width 0.25) (layer "F.Cu") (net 24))
 (segment (start 15.7 1.5) (end 15.7 3.6) (width 0.25) (layer "F.Cu") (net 21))
 (segment (start 17.056 4.956) (end 19.25 4.956) (width 0.25) (layer "F.Cu") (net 21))
 (segment (start 15.7 3.6) (end 17.056 4.956) (width 0.25) (layer "F.Cu") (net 21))
 (segment (start 4.3304 9.3429) (end 4.3875 9.4) (width 0.25) (layer "F.Cu") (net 23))
 (segment (start 1.7 9.3429) (end 4.3304 9.3429) (width 0.25) (layer "F.Cu") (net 23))
 (segment (start 4.3446 11.3571) (end 4.3875 11.4) (width 0.25) (layer "F.Cu") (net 20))
 (segment (start 1.7 11.3571) (end 4.3446 11.3571) (width 0.25) (layer "F.Cu") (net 20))
 (segment (start 1.7 13.3714) (end 4.3339 13.3714) (width 0.25) (layer "F.Cu") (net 19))
 (segment (start 4.3339 13.3714) (end 4.3625 13.4) (width 0.25) (layer "F.Cu") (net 19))
 (segment (start 4.3732 15.3857) (end 4.3875 15.4) (width 0.25) (layer "F.Cu") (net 25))
 (segment (start 1.7 15.3857) (end 4.3732 15.3857) (width 0.25) (layer "F.Cu") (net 25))
 (segment (start 1.7 17.4) (end 4.3875 17.4) (width 0.25) (layer "F.Cu") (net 22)))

